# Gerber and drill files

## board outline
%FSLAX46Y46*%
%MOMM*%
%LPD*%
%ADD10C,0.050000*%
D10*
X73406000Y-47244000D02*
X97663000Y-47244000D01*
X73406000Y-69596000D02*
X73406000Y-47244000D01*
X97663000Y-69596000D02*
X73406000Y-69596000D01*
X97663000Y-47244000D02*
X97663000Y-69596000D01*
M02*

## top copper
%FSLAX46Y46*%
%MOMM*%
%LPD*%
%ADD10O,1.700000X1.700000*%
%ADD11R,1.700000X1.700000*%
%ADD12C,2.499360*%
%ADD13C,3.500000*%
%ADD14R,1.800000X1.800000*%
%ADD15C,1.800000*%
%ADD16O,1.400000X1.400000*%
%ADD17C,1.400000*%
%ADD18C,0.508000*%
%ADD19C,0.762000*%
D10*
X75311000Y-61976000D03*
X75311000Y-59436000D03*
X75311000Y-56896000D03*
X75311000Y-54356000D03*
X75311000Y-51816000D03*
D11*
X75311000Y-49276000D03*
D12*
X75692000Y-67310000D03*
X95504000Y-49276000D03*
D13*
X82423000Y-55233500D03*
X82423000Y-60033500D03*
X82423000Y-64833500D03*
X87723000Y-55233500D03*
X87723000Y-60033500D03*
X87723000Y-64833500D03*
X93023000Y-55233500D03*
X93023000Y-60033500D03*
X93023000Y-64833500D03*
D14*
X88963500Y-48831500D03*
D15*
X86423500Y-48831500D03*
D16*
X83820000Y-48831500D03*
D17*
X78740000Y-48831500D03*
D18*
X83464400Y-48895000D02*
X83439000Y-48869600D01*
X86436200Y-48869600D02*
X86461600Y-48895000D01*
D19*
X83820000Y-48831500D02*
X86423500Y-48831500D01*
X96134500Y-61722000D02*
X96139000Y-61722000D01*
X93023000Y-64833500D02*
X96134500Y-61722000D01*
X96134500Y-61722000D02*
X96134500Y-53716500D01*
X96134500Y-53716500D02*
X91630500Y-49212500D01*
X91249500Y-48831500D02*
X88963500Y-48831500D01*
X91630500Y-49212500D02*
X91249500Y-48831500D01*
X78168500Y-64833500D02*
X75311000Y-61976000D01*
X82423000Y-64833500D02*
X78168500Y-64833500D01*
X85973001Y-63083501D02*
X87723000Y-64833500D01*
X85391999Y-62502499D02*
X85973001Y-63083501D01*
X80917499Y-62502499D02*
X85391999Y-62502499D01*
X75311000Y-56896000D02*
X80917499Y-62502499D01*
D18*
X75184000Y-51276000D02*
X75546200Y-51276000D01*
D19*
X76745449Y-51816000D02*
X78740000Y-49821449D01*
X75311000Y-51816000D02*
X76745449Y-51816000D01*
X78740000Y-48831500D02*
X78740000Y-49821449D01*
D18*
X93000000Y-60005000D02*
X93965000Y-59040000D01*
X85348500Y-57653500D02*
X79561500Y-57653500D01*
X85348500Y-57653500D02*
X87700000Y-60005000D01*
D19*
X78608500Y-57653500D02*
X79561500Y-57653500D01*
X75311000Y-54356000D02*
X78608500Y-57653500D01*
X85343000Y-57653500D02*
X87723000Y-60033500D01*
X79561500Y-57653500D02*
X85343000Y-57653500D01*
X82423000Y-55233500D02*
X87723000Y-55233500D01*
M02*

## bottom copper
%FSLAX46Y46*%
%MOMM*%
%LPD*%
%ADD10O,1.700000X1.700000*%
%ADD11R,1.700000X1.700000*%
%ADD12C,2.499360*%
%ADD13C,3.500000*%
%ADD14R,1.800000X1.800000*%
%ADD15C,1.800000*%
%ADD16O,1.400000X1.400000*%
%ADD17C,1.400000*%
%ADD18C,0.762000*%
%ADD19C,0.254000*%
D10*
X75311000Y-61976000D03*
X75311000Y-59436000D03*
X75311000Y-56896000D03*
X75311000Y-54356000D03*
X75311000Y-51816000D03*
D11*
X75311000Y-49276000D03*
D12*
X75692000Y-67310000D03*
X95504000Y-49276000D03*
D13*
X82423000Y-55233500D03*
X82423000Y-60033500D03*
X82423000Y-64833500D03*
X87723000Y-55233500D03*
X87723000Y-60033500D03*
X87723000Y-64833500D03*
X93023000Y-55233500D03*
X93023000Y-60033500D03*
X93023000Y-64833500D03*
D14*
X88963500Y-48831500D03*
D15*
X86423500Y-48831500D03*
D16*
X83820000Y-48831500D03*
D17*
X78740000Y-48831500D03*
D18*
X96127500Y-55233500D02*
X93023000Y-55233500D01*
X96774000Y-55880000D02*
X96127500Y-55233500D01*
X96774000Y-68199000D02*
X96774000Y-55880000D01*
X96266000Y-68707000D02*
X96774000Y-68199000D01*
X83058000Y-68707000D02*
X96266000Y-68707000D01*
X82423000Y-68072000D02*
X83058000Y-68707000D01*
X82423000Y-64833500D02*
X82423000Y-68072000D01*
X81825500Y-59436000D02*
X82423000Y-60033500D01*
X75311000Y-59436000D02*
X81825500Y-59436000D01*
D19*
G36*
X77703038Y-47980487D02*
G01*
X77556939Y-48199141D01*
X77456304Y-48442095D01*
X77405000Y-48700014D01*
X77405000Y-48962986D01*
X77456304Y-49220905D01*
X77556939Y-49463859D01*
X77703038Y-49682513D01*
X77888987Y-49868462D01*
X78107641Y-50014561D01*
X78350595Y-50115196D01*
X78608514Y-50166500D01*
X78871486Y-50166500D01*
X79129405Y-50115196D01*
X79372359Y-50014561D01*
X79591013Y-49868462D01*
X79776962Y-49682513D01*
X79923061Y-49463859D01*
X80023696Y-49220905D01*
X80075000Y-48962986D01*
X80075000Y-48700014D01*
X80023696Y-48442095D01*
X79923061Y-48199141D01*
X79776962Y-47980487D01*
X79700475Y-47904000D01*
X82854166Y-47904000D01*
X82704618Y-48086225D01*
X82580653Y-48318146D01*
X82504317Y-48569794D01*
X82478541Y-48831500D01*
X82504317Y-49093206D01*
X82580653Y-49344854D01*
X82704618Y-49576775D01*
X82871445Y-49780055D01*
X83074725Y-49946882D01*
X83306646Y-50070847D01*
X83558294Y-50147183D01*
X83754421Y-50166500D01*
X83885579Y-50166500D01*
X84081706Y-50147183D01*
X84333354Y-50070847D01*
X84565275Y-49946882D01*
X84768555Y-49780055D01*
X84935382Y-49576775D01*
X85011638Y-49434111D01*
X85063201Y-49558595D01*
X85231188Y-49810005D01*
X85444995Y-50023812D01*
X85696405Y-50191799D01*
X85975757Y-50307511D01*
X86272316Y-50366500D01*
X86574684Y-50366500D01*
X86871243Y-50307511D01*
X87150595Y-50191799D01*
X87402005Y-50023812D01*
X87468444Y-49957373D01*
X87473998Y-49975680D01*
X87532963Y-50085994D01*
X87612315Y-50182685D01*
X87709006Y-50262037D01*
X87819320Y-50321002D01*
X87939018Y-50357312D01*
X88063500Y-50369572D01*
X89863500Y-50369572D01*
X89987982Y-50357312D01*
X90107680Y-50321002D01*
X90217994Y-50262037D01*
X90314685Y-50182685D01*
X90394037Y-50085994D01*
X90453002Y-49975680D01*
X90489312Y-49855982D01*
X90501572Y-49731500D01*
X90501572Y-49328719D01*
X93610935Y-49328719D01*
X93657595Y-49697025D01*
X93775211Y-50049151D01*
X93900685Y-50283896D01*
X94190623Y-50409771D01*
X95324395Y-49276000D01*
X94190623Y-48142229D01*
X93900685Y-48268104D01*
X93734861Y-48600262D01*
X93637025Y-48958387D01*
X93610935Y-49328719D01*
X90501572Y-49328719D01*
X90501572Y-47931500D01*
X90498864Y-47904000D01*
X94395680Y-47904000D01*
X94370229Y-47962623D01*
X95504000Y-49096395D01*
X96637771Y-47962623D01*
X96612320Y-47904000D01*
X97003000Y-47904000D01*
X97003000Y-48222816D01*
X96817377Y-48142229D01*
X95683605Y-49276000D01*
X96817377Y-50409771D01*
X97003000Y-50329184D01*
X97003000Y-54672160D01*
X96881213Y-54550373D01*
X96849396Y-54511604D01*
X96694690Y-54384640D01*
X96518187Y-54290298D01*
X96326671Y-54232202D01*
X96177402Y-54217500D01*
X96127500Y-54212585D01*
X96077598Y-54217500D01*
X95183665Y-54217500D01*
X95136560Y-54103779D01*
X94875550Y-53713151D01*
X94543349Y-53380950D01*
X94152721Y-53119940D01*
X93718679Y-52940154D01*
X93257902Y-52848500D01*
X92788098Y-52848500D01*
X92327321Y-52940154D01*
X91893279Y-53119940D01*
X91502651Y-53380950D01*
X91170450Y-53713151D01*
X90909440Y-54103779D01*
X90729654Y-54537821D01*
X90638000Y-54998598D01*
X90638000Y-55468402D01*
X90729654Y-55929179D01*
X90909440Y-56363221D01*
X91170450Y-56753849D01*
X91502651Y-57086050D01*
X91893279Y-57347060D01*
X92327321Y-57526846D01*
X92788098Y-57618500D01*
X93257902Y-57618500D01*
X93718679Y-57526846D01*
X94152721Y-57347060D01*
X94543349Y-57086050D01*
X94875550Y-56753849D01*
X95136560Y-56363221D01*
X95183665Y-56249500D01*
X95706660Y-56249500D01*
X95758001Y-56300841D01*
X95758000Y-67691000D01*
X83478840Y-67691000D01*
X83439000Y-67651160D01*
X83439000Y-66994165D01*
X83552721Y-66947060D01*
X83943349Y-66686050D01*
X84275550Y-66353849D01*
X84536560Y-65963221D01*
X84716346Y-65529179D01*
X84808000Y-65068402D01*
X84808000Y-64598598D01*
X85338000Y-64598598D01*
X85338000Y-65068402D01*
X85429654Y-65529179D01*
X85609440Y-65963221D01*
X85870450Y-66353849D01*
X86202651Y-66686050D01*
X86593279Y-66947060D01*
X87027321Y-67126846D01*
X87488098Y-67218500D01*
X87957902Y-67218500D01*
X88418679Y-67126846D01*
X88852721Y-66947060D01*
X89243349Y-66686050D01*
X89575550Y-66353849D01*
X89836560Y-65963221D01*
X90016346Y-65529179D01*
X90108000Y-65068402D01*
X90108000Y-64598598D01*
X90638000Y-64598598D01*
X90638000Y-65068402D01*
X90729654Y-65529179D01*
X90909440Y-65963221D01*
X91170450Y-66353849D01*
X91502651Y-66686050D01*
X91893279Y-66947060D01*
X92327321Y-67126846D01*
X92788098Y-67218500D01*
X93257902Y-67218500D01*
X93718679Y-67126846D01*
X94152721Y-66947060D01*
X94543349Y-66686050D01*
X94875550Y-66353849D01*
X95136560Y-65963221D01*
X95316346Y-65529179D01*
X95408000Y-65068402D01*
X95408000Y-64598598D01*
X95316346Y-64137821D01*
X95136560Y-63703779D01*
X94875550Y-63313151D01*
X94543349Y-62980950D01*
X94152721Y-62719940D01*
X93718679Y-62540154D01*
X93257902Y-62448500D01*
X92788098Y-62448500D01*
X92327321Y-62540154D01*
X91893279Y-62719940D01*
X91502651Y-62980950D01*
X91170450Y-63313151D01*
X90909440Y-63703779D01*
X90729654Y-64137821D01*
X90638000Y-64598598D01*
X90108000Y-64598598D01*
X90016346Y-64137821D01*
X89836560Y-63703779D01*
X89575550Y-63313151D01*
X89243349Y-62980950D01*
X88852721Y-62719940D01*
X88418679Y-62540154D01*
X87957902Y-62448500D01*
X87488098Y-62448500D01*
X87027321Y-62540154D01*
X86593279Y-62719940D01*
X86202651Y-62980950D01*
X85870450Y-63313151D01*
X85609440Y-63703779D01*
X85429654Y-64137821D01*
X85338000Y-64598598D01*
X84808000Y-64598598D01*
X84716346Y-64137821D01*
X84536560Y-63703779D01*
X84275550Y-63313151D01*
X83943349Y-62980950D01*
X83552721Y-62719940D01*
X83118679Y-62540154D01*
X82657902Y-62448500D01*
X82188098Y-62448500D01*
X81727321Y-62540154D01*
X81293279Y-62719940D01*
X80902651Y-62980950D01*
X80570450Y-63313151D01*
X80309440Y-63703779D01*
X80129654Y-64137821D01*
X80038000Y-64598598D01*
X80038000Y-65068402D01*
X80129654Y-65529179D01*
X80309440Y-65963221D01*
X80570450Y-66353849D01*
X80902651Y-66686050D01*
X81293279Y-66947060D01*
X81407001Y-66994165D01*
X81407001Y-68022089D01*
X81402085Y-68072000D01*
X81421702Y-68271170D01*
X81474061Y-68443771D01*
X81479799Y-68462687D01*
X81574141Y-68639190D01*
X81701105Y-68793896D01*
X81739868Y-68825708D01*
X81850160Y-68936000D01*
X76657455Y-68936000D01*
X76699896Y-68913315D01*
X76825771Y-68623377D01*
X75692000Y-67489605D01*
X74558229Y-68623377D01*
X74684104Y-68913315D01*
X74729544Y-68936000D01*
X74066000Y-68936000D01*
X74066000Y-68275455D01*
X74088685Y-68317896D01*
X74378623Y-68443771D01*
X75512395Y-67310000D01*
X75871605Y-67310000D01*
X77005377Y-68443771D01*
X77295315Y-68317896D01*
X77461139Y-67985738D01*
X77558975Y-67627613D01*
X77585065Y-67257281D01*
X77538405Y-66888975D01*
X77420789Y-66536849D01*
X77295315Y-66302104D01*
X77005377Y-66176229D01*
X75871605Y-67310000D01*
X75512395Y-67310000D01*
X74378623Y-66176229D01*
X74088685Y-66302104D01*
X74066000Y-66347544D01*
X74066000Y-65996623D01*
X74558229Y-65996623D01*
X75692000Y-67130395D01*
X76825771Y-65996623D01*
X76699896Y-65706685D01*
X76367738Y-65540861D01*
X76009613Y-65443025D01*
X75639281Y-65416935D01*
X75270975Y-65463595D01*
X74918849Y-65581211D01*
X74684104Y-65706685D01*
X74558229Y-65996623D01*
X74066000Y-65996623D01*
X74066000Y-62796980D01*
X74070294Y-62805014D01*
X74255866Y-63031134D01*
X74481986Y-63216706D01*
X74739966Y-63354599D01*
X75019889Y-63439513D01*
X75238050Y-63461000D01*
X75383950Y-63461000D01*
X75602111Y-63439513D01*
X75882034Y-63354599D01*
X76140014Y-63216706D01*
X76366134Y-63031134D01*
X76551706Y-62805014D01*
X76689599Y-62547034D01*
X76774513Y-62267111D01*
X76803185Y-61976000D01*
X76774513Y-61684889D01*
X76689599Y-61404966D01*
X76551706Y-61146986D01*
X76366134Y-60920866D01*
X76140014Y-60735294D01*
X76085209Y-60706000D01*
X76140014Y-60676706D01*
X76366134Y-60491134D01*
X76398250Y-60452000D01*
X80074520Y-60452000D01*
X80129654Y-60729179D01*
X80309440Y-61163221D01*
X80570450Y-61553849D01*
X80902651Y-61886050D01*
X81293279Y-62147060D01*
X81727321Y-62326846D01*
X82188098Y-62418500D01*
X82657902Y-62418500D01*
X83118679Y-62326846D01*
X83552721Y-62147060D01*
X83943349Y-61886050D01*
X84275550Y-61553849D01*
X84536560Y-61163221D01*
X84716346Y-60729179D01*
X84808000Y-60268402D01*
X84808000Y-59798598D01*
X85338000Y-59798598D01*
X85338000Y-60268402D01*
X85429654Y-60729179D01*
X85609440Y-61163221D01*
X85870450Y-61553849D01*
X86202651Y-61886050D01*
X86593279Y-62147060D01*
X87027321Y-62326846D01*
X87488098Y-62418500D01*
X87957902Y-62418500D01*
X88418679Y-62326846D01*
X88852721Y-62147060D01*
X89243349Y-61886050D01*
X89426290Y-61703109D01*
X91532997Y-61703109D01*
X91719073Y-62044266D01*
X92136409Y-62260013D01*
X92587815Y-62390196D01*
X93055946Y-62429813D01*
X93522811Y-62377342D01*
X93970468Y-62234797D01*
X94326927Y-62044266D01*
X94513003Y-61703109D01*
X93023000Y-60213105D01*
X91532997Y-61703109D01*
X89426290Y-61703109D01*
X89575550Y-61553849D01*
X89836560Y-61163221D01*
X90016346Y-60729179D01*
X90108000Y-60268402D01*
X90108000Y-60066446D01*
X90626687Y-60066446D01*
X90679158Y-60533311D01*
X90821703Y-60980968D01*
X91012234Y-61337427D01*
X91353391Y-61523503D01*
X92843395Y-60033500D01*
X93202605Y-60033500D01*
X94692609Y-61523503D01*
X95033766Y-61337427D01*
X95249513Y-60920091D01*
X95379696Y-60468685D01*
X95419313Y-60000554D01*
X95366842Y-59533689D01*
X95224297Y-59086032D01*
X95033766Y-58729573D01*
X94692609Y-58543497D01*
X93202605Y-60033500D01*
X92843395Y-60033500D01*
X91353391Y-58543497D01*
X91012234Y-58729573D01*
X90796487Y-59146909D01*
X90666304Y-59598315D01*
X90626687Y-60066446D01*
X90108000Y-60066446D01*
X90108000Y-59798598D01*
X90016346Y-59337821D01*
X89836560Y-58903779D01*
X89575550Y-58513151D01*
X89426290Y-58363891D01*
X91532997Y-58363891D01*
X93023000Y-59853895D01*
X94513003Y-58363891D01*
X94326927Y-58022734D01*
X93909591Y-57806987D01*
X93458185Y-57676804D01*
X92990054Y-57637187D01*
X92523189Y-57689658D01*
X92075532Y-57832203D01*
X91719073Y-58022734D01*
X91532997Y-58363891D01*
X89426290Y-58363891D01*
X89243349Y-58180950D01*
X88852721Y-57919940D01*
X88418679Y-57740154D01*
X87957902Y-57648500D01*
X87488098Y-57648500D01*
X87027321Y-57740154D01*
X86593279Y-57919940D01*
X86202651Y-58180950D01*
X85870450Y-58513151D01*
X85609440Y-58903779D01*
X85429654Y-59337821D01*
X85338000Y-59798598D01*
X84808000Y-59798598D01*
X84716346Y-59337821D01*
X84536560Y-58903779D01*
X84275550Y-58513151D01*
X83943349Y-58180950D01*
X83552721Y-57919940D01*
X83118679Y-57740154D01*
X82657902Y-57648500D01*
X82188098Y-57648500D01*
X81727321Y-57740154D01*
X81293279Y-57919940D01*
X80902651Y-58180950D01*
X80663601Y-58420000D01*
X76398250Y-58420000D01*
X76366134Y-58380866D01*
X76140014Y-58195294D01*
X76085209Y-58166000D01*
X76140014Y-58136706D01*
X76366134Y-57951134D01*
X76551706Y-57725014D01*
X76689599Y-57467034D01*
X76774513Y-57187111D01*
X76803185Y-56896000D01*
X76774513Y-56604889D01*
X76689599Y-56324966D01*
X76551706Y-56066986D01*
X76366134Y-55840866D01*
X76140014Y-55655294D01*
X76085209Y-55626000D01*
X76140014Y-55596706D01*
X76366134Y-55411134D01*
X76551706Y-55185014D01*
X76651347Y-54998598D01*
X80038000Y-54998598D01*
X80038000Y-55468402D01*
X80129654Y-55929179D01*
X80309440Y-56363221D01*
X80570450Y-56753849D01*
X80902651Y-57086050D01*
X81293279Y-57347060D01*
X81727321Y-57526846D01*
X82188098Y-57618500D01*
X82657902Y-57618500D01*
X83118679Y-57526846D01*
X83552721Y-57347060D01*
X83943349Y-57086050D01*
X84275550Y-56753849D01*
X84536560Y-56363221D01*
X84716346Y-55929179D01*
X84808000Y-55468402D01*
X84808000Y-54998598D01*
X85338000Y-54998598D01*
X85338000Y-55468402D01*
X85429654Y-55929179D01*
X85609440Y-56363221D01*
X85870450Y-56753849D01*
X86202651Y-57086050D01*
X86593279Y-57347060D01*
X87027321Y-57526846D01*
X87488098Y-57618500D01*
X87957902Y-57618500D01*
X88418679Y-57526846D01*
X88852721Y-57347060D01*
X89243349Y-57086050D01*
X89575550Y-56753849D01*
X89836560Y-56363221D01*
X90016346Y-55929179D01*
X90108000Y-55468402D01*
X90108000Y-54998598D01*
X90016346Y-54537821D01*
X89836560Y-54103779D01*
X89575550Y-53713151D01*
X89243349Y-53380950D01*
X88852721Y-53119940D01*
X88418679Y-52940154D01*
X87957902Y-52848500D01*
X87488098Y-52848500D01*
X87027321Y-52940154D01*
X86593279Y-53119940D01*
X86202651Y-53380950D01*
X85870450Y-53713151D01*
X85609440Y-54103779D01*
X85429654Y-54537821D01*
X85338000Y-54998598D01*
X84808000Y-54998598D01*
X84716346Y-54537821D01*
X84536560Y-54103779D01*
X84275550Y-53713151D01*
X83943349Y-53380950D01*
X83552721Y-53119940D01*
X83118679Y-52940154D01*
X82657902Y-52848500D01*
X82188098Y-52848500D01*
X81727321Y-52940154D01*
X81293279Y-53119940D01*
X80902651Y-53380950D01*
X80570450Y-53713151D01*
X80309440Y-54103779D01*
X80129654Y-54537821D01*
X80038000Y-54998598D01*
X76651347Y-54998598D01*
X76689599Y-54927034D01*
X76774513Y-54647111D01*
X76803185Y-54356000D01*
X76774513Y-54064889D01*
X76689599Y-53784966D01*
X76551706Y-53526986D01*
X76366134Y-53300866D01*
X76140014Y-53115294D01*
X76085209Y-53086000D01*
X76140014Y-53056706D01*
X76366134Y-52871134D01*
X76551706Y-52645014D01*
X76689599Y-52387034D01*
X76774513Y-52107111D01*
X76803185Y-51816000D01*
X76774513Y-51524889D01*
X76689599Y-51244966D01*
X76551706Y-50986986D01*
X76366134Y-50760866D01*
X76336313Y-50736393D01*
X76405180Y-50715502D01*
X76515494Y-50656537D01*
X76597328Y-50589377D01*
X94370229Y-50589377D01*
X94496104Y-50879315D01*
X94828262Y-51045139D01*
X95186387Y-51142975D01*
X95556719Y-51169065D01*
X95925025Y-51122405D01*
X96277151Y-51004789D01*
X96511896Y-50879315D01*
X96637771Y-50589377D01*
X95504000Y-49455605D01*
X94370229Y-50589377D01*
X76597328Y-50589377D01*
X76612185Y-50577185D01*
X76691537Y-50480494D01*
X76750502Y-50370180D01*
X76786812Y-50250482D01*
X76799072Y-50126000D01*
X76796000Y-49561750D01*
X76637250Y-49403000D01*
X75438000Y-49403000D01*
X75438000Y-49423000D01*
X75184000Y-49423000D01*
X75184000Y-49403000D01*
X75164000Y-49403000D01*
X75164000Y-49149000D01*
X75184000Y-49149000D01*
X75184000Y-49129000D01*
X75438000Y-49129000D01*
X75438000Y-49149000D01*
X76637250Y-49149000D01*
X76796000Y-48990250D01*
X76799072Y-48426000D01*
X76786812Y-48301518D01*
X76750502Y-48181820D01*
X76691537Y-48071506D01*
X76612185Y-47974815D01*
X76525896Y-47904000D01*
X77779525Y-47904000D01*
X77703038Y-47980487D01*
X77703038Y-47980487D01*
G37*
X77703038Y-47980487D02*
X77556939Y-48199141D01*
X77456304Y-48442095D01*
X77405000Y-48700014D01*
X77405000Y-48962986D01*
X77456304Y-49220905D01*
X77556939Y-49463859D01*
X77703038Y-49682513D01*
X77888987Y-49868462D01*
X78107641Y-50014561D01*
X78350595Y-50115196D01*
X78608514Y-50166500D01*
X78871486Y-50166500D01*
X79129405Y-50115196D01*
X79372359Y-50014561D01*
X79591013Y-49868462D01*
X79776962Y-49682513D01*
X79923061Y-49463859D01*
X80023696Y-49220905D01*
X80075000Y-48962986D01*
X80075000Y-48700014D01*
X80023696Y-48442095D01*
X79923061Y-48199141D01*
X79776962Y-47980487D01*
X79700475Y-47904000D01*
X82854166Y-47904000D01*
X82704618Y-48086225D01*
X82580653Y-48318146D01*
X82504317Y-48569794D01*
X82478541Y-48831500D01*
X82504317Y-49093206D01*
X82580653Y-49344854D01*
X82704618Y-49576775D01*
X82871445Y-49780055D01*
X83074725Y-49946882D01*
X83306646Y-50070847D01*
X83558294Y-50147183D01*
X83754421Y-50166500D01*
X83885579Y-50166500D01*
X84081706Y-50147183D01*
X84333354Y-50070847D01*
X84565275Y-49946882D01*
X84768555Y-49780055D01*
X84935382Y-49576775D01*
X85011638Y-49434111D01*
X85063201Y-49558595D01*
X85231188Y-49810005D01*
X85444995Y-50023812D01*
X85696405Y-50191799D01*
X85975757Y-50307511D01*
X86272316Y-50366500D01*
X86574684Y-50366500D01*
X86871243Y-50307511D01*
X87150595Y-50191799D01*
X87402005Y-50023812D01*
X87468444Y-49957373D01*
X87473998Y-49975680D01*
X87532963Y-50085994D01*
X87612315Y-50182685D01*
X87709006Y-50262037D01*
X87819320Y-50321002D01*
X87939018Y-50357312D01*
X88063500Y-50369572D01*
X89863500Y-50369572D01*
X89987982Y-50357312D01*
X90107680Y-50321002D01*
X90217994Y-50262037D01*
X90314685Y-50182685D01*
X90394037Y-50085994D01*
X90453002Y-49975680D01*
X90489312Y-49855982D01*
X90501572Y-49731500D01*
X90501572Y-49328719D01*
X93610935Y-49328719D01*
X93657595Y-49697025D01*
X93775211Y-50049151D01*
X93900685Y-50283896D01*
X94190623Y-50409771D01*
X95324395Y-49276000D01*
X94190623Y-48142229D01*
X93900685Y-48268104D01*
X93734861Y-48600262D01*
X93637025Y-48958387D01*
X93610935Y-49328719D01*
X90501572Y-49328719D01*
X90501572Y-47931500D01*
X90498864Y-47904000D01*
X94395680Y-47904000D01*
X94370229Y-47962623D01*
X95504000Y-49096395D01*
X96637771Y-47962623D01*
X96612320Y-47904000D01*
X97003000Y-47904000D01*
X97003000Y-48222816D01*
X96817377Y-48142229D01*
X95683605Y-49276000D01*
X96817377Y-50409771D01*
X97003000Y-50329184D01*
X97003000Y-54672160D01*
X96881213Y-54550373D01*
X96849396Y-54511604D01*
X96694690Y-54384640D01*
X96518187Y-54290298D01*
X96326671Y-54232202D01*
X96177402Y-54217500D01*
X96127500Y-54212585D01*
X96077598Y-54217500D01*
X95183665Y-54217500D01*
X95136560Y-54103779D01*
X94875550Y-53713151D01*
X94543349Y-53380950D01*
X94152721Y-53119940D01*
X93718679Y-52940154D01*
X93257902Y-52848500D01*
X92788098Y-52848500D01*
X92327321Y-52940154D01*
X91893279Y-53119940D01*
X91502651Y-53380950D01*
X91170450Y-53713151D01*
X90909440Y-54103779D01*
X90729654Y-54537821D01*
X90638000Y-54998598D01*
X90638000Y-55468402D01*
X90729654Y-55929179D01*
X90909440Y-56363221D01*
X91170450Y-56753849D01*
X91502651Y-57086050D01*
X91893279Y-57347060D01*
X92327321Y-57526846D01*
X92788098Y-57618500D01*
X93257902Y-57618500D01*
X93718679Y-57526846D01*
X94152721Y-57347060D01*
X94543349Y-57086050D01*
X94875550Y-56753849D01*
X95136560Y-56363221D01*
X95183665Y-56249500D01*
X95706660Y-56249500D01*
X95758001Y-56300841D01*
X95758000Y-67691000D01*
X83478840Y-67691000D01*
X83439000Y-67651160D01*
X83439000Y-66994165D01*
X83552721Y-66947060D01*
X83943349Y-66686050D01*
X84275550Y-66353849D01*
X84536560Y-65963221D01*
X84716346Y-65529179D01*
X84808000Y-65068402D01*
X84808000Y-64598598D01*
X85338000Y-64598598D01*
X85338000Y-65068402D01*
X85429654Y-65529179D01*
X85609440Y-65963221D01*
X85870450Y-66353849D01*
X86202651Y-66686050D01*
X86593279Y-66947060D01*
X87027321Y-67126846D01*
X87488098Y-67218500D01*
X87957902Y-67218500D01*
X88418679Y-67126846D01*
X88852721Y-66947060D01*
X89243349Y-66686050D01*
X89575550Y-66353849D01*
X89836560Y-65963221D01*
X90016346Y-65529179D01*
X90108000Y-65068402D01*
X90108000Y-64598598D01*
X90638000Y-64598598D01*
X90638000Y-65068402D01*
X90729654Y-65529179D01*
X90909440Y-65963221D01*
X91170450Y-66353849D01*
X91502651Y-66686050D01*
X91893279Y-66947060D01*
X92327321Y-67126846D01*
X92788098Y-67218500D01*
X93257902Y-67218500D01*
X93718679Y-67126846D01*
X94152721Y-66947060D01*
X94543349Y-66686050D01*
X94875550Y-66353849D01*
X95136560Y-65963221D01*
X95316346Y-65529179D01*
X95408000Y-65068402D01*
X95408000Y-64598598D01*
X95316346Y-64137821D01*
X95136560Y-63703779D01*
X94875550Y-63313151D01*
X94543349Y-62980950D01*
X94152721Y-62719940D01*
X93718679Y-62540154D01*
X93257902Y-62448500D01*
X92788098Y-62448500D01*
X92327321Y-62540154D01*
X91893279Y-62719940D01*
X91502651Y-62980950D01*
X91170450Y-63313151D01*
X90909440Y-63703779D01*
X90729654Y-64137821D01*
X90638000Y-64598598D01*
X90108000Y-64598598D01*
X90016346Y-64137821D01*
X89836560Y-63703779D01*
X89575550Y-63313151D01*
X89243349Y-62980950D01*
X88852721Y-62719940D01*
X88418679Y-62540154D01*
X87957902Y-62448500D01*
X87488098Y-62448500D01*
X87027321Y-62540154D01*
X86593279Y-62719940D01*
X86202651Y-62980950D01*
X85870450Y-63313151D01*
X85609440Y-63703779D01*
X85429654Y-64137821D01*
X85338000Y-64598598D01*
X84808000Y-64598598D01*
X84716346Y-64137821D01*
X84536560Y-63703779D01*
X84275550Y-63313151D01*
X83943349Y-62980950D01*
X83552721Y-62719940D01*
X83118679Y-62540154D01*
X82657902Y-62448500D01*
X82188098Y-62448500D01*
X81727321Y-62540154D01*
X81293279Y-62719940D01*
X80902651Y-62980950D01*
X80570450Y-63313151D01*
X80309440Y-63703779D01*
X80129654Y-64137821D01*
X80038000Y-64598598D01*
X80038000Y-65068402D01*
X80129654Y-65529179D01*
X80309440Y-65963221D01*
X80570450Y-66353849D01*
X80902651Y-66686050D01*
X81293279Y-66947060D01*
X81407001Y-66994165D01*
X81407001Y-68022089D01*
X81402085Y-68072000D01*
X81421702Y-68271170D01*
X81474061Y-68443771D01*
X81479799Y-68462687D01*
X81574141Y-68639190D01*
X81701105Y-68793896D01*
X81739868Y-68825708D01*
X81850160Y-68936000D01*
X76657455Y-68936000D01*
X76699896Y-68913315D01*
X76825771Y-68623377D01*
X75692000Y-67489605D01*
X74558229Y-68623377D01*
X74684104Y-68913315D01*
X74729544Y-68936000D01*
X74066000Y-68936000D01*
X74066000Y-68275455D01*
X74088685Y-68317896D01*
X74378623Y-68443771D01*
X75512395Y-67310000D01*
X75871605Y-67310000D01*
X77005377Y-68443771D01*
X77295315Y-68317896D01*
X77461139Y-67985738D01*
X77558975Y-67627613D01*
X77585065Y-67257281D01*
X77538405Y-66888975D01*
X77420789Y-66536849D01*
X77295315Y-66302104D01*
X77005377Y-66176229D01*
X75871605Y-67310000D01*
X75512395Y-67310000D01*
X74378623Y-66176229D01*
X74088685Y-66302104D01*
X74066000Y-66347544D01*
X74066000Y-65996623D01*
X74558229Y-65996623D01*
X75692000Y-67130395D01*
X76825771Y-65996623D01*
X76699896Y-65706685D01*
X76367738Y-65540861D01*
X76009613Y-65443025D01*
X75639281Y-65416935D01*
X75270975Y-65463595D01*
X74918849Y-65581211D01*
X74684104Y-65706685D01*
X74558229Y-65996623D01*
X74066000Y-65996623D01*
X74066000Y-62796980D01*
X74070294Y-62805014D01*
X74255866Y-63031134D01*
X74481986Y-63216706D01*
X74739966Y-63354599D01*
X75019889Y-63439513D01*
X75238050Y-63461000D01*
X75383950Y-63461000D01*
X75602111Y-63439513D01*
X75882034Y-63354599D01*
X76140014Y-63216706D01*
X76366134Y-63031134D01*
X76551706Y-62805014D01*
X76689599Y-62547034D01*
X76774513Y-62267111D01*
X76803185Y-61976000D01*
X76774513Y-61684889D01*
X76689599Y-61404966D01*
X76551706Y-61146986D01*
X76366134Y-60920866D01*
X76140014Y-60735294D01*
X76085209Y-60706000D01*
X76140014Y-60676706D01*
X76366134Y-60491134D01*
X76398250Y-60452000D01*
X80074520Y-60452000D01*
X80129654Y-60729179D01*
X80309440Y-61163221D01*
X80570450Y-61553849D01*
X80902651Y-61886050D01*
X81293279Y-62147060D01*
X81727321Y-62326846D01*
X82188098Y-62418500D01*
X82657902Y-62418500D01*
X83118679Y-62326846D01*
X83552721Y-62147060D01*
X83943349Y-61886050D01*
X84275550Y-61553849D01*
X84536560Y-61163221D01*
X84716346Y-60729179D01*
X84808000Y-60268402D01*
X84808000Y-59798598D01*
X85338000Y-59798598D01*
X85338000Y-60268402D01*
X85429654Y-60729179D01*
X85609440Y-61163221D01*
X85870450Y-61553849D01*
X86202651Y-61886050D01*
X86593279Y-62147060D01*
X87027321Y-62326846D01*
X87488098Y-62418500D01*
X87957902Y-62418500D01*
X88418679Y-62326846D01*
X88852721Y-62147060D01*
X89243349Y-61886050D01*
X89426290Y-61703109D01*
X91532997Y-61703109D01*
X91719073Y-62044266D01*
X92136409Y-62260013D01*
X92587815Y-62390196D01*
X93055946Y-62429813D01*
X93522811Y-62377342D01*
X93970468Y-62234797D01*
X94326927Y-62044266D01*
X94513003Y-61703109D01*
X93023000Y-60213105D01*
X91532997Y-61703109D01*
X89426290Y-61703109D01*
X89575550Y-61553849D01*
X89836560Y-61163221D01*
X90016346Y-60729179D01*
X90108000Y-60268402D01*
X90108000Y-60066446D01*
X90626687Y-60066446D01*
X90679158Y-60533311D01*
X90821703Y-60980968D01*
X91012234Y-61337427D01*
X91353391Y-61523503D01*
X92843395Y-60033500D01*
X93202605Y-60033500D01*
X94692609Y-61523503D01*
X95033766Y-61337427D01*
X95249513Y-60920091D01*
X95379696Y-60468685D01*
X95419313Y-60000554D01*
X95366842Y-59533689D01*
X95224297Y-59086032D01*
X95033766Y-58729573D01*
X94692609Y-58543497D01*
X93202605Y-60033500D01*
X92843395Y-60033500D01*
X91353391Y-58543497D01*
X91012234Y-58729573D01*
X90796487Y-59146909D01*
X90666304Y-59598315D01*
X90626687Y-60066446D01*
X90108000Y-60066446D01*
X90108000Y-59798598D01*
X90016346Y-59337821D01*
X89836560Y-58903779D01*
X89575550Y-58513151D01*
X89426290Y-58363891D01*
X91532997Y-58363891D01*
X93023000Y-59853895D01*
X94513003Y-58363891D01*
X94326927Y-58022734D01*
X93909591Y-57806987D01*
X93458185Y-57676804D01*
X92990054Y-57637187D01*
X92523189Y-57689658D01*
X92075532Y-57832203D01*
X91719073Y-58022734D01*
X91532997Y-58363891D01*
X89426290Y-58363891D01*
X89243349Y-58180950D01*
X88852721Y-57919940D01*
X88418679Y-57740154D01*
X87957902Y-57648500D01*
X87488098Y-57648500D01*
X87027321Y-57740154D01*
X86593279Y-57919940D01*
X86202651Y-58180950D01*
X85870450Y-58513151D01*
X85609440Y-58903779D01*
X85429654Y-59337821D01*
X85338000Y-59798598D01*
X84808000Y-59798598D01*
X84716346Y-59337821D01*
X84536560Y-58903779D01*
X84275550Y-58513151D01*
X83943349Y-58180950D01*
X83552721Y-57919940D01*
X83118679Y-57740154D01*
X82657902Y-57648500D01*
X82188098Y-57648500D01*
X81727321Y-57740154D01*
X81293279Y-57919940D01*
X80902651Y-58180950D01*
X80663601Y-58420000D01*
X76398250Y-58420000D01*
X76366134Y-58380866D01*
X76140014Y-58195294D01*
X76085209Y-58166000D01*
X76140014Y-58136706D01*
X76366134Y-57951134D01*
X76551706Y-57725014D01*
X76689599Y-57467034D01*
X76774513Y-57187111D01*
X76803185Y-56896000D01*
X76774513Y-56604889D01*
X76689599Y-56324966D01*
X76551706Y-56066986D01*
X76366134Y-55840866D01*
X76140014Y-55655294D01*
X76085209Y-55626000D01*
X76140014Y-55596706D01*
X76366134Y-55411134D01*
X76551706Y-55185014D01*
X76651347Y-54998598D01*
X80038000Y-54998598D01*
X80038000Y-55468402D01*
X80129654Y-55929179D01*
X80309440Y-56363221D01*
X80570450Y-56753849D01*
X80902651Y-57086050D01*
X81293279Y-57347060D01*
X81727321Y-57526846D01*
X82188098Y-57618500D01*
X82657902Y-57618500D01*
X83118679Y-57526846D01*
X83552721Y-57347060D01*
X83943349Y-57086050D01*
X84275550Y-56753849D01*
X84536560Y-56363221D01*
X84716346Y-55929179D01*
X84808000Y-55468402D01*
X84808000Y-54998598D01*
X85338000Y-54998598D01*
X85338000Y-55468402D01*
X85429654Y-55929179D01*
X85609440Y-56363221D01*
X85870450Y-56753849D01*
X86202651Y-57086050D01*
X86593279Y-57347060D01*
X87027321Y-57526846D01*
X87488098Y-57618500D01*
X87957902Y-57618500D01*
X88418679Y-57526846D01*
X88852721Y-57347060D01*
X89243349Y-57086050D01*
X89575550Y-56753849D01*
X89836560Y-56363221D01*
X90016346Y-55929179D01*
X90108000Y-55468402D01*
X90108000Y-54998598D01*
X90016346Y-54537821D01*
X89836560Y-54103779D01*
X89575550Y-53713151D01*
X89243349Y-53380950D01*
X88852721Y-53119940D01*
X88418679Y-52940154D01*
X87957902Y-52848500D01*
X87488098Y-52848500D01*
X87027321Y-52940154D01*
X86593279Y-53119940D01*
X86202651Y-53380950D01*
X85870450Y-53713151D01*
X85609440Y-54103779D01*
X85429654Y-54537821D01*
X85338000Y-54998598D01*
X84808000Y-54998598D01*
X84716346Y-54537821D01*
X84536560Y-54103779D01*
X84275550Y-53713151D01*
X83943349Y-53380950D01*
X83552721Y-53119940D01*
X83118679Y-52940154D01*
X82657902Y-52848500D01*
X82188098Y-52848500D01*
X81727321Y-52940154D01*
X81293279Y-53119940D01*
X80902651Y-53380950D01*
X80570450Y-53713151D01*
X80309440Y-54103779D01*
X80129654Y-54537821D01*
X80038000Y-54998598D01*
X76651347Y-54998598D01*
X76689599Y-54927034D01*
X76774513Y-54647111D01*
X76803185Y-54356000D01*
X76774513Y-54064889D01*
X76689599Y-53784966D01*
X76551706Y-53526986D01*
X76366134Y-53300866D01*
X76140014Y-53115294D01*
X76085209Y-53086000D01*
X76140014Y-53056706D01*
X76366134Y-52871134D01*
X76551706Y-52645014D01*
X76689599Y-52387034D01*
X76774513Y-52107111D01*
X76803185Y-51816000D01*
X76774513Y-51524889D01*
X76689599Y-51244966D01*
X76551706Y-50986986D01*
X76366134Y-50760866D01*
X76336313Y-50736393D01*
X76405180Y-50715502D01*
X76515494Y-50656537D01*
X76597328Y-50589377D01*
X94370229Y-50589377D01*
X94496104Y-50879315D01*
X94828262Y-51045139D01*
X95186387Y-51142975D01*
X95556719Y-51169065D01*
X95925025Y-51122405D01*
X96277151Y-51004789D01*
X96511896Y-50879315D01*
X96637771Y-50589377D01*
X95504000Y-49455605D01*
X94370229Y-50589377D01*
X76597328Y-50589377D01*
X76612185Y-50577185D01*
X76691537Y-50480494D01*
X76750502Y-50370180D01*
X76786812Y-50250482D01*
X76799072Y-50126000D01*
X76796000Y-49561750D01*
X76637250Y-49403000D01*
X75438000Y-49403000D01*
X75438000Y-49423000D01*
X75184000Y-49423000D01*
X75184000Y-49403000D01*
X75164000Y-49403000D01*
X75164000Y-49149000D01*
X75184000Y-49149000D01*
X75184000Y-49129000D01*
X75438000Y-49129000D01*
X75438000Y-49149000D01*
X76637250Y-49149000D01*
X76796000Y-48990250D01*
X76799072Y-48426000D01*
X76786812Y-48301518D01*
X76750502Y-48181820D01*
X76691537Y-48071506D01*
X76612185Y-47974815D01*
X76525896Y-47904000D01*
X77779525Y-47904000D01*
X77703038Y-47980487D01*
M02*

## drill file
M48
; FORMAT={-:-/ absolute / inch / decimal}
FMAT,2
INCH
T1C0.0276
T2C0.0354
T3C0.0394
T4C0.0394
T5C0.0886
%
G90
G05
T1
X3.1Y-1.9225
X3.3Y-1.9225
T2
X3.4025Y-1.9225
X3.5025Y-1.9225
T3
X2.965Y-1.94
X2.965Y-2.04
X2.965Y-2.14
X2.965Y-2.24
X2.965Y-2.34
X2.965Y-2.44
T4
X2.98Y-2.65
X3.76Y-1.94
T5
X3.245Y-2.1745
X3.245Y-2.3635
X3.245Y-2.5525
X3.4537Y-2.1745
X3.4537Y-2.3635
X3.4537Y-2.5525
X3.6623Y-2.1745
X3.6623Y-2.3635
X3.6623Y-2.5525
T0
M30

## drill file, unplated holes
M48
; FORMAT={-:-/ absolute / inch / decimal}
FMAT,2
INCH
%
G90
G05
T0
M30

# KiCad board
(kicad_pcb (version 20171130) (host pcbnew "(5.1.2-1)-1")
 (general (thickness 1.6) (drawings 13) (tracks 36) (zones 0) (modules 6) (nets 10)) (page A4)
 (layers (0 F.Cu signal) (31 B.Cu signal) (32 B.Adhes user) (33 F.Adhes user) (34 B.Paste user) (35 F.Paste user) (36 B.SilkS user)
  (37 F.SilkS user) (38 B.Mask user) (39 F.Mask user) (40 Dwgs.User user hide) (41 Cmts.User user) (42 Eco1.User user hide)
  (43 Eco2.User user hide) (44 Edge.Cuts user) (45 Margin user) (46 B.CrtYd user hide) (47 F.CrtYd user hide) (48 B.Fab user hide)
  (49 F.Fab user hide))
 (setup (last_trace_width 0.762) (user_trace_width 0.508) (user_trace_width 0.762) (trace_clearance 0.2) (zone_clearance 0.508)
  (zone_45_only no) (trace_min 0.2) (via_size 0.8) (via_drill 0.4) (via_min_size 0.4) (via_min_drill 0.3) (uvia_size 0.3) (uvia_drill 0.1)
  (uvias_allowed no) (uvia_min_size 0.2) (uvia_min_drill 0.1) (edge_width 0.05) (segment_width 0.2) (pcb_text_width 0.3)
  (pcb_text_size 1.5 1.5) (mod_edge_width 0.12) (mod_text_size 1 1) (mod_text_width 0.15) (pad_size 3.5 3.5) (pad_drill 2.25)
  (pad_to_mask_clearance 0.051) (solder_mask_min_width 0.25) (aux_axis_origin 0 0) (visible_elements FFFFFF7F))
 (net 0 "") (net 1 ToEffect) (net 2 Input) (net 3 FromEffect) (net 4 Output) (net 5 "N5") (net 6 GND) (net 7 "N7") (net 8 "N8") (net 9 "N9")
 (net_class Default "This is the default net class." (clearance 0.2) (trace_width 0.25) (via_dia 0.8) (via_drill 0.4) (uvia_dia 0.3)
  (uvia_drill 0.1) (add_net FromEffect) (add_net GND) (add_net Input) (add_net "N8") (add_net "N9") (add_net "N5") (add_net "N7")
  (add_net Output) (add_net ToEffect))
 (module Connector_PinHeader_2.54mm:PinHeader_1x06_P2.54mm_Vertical (layer F.Cu) (at 75.311 49.276)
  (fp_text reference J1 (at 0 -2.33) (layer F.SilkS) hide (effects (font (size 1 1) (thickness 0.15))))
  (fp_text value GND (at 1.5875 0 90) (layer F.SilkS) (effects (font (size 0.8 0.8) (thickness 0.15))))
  (pad 6 thru_hole oval (at 0 12.7) (size 1.7 1.7) (drill 1) (layers *.Cu *.Mask) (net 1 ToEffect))
  (pad 5 thru_hole oval (at 0 10.16) (size 1.7 1.7) (drill 1) (layers *.Cu *.Mask) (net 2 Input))
  (pad 4 thru_hole oval (at 0 7.62) (size 1.7 1.7) (drill 1) (layers *.Cu *.Mask) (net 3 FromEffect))
  (pad 3 thru_hole oval (at 0 5.08) (size 1.7 1.7) (drill 1) (layers *.Cu *.Mask) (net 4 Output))
  (pad 2 thru_hole oval (at 0 2.54) (size 1.7 1.7) (drill 1) (layers *.Cu *.Mask) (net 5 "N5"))
  (pad 1 thru_hole rect (at 0 0) (size 1.7 1.7) (drill 1) (layers *.Cu *.Mask) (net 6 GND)))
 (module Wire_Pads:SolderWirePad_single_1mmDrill (layer F.Cu) (at 75.692 67.31)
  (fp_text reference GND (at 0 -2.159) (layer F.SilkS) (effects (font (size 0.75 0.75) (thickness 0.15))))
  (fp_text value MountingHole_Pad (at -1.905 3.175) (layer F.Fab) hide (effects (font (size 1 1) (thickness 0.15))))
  (pad 1 thru_hole circle (at 0 0) (size 2.49936 2.49936) (drill 1.00076) (layers *.Cu *.Mask) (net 6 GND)))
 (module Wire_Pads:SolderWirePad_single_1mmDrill (layer F.Cu) (at 95.504 49.276)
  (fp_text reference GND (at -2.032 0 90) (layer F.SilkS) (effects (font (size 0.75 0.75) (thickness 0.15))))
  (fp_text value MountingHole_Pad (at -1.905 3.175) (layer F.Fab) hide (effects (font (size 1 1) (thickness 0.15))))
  (pad 1 thru_hole circle (at 0 0) (size 2.49936 2.49936) (drill 1.00076) (layers *.Cu *.Mask) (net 6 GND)))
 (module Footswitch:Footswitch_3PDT (layer F.Cu) (at 87.723 60.0335)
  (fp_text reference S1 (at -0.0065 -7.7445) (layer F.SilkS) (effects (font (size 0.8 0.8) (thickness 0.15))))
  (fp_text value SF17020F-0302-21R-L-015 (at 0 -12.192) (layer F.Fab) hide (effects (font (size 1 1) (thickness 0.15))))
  (pad 9 thru_hole circle (at -5.3 -4.8 90) (size 3.5 3.5) (drill 2.25) (layers *.Cu *.Mask F.SilkS) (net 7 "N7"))
  (pad 8 thru_hole circle (at -5.3 0 90) (size 3.5 3.5) (drill 2.25) (layers *.Cu *.Mask F.SilkS) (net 2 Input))
  (pad 7 thru_hole circle (at -5.3 4.8 90) (size 3.5 3.5) (drill 2.25) (layers *.Cu *.Mask F.SilkS) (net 1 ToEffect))
  (pad 6 thru_hole circle (at 0 -4.8 90) (size 3.5 3.5) (drill 2.25) (layers *.Cu *.Mask F.SilkS) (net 7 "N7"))
  (pad 5 thru_hole circle (at 0 0 90) (size 3.5 3.5) (drill 2.25) (layers *.Cu *.Mask F.SilkS) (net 4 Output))
  (pad 4 thru_hole circle (at 0 4.8 90) (size 3.5 3.5) (drill 2.25) (layers *.Cu *.Mask F.SilkS) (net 3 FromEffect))
  (pad 3 thru_hole circle (at 5.3 -4.8 90) (size 3.5 3.5) (drill 2.25) (layers *.Cu *.Mask F.SilkS) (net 1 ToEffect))
  (pad 2 thru_hole circle (at 5.3 0 90) (size 3.5 3.5) (drill 2.25) (layers *.Cu *.Mask F.SilkS) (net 6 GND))
  (pad 1 thru_hole circle (at 5.3 4.8 90) (size 3.5 3.5) (drill 2.25) (layers *.Cu *.Mask F.SilkS) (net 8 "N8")))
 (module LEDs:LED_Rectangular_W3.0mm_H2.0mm (layer F.Cu) (at 88.9635 48.8315 180)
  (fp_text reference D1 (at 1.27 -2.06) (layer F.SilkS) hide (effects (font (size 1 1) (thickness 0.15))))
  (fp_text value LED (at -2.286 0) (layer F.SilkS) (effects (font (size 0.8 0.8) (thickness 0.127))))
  (pad 1 thru_hole rect (at 0 0 180) (size 1.8 1.8) (drill 0.9) (layers *.Cu *.Mask) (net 8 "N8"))
  (pad 2 thru_hole circle (at 2.54 0 180) (size 1.8 1.8) (drill 0.9) (layers *.Cu *.Mask) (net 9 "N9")))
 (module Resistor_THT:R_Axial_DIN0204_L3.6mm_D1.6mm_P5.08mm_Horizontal (layer F.Cu) (at 78.74 48.8315)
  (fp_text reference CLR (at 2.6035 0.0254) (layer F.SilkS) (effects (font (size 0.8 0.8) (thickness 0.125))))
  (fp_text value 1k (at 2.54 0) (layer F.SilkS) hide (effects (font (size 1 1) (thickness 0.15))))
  (pad 2 thru_hole oval (at 5.08 0) (size 1.4 1.4) (drill 0.7) (layers *.Cu *.Mask) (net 9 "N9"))
  (pad 1 thru_hole circle (at 0 0) (size 1.4 1.4) (drill 0.7) (layers *.Cu *.Mask) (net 5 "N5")))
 (gr_line (start 73.406 47.244) (end 97.663 47.244) (layer Edge.Cuts) (width 0.05))
 (gr_line (start 73.406 69.596) (end 73.406 47.244) (layer Edge.Cuts) (width 0.05))
 (gr_line (start 97.663 69.596) (end 73.406 69.596) (layer Edge.Cuts) (width 0.05))
 (gr_line (start 97.663 47.244) (end 97.663 69.596) (layer Edge.Cuts) (width 0.05))
 (segment (start 83.4644 48.895) (end 83.439 48.8696) (width 0.508) (layer F.Cu) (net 9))
 (segment (start 86.4362 48.8696) (end 86.4616 48.895) (width 0.508) (layer F.Cu) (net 9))
 (segment (start 83.82 48.8315) (end 86.4235 48.8315) (width 0.762) (layer F.Cu) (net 9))
 (segment (start 96.1345 61.722) (end 96.139 61.722) (width 0.762) (layer F.Cu) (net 8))
 (segment (start 93.023 64.8335) (end 96.1345 61.722) (width 0.762) (layer F.Cu) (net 8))
 (segment (start 96.1345 61.722) (end 96.1345 53.7165) (width 0.762) (layer F.Cu) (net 8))
 (segment (start 96.1345 53.7165) (end 91.6305 49.2125) (width 0.762) (layer F.Cu) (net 8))
 (segment (start 91.2495 48.8315) (end 88.9635 48.8315) (width 0.762) (layer F.Cu) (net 8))
 (segment (start 91.6305 49.2125) (end 91.2495 48.8315) (width 0.762) (layer F.Cu) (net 8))
 (segment (start 96.1275 55.2335) (end 93.023 55.2335) (width 0.762) (layer B.Cu) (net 1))
 (segment (start 96.774 55.88) (end 96.1275 55.2335) (width 0.762) (layer B.Cu) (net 1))
 (segment (start 96.774 68.199) (end 96.774 55.88) (width 0.762) (layer B.Cu) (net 1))
 (segment (start 96.266 68.707) (end 96.774 68.199) (width 0.762) (layer B.Cu) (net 1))
 (segment (start 83.058 68.707) (end 96.266 68.707) (width 0.762) (layer B.Cu) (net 1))
 (segment (start 82.423 68.072) (end 83.058 68.707) (width 0.762) (layer B.Cu) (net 1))
 (segment (start 82.423 64.8335) (end 82.423 68.072) (width 0.762) (layer B.Cu) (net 1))
 (segment (start 78.1685 64.8335) (end 75.311 61.976) (width 0.762) (layer F.Cu) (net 1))
 (segment (start 82.423 64.8335) (end 78.1685 64.8335) (width 0.762) (layer F.Cu) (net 1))
 (segment (start 81.8255 59.436) (end 82.423 60.0335) (width 0.762) (layer B.Cu) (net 2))
 (segment (start 75.311 59.436) (end 81.8255 59.436) (width 0.762) (layer B.Cu) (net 2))
 (segment (start 85.973001 63.083501) (end 87.723 64.8335) (width 0.762) (layer F.Cu) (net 3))
 (segment (start 85.391999 62.502499) (end 85.973001 63.083501) (width 0.762) (layer F.Cu) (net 3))
 (segment (start 80.917499 62.502499) (end 85.391999 62.502499) (width 0.762) (layer F.Cu) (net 3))
 (segment (start 75.311 56.896) (end 80.917499 62.502499) (width 0.762) (layer F.Cu) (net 3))
 (segment (start 75.184 51.276) (end 75.5462 51.276) (width 0.508) (layer F.Cu) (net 5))
 (segment (start 76.745449 51.816) (end 78.74 49.821449) (width 0.762) (layer F.Cu) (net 5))
 (segment (start 75.311 51.816) (end 76.745449 51.816) (width 0.762) (layer F.Cu) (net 5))
 (segment (start 78.74 48.8315) (end 78.74 49.821449) (width 0.762) (layer F.Cu) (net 5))
 (segment (start 93 60.005) (end 93.965 59.04) (width 0.508) (layer F.Cu) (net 6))
 (segment (start 85.3485 57.6535) (end 79.5615 57.6535) (width 0.508) (layer F.Cu) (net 4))
 (segment (start 85.3485 57.6535) (end 87.7 60.005) (width 0.508) (layer F.Cu) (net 4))
 (segment (start 78.6085 57.6535) (end 79.5615 57.6535) (width 0.762) (layer F.Cu) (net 4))
 (segment (start 75.311 54.356) (end 78.6085 57.6535) (width 0.762) (layer F.Cu) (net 4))
 (segment (start 85.343 57.6535) (end 87.723 60.0335) (width 0.762) (layer F.Cu) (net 4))
 (segment (start 79.5615 57.6535) (end 85.343 57.6535) (width 0.762) (layer F.Cu) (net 4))
 (segment (start 82.423 55.2335) (end 87.723 55.2335) (width 0.762) (layer F.Cu) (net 7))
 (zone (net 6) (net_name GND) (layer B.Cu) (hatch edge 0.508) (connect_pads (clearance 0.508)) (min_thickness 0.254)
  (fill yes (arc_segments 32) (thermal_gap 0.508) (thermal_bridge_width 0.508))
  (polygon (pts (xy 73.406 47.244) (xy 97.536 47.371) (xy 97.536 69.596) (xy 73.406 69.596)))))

